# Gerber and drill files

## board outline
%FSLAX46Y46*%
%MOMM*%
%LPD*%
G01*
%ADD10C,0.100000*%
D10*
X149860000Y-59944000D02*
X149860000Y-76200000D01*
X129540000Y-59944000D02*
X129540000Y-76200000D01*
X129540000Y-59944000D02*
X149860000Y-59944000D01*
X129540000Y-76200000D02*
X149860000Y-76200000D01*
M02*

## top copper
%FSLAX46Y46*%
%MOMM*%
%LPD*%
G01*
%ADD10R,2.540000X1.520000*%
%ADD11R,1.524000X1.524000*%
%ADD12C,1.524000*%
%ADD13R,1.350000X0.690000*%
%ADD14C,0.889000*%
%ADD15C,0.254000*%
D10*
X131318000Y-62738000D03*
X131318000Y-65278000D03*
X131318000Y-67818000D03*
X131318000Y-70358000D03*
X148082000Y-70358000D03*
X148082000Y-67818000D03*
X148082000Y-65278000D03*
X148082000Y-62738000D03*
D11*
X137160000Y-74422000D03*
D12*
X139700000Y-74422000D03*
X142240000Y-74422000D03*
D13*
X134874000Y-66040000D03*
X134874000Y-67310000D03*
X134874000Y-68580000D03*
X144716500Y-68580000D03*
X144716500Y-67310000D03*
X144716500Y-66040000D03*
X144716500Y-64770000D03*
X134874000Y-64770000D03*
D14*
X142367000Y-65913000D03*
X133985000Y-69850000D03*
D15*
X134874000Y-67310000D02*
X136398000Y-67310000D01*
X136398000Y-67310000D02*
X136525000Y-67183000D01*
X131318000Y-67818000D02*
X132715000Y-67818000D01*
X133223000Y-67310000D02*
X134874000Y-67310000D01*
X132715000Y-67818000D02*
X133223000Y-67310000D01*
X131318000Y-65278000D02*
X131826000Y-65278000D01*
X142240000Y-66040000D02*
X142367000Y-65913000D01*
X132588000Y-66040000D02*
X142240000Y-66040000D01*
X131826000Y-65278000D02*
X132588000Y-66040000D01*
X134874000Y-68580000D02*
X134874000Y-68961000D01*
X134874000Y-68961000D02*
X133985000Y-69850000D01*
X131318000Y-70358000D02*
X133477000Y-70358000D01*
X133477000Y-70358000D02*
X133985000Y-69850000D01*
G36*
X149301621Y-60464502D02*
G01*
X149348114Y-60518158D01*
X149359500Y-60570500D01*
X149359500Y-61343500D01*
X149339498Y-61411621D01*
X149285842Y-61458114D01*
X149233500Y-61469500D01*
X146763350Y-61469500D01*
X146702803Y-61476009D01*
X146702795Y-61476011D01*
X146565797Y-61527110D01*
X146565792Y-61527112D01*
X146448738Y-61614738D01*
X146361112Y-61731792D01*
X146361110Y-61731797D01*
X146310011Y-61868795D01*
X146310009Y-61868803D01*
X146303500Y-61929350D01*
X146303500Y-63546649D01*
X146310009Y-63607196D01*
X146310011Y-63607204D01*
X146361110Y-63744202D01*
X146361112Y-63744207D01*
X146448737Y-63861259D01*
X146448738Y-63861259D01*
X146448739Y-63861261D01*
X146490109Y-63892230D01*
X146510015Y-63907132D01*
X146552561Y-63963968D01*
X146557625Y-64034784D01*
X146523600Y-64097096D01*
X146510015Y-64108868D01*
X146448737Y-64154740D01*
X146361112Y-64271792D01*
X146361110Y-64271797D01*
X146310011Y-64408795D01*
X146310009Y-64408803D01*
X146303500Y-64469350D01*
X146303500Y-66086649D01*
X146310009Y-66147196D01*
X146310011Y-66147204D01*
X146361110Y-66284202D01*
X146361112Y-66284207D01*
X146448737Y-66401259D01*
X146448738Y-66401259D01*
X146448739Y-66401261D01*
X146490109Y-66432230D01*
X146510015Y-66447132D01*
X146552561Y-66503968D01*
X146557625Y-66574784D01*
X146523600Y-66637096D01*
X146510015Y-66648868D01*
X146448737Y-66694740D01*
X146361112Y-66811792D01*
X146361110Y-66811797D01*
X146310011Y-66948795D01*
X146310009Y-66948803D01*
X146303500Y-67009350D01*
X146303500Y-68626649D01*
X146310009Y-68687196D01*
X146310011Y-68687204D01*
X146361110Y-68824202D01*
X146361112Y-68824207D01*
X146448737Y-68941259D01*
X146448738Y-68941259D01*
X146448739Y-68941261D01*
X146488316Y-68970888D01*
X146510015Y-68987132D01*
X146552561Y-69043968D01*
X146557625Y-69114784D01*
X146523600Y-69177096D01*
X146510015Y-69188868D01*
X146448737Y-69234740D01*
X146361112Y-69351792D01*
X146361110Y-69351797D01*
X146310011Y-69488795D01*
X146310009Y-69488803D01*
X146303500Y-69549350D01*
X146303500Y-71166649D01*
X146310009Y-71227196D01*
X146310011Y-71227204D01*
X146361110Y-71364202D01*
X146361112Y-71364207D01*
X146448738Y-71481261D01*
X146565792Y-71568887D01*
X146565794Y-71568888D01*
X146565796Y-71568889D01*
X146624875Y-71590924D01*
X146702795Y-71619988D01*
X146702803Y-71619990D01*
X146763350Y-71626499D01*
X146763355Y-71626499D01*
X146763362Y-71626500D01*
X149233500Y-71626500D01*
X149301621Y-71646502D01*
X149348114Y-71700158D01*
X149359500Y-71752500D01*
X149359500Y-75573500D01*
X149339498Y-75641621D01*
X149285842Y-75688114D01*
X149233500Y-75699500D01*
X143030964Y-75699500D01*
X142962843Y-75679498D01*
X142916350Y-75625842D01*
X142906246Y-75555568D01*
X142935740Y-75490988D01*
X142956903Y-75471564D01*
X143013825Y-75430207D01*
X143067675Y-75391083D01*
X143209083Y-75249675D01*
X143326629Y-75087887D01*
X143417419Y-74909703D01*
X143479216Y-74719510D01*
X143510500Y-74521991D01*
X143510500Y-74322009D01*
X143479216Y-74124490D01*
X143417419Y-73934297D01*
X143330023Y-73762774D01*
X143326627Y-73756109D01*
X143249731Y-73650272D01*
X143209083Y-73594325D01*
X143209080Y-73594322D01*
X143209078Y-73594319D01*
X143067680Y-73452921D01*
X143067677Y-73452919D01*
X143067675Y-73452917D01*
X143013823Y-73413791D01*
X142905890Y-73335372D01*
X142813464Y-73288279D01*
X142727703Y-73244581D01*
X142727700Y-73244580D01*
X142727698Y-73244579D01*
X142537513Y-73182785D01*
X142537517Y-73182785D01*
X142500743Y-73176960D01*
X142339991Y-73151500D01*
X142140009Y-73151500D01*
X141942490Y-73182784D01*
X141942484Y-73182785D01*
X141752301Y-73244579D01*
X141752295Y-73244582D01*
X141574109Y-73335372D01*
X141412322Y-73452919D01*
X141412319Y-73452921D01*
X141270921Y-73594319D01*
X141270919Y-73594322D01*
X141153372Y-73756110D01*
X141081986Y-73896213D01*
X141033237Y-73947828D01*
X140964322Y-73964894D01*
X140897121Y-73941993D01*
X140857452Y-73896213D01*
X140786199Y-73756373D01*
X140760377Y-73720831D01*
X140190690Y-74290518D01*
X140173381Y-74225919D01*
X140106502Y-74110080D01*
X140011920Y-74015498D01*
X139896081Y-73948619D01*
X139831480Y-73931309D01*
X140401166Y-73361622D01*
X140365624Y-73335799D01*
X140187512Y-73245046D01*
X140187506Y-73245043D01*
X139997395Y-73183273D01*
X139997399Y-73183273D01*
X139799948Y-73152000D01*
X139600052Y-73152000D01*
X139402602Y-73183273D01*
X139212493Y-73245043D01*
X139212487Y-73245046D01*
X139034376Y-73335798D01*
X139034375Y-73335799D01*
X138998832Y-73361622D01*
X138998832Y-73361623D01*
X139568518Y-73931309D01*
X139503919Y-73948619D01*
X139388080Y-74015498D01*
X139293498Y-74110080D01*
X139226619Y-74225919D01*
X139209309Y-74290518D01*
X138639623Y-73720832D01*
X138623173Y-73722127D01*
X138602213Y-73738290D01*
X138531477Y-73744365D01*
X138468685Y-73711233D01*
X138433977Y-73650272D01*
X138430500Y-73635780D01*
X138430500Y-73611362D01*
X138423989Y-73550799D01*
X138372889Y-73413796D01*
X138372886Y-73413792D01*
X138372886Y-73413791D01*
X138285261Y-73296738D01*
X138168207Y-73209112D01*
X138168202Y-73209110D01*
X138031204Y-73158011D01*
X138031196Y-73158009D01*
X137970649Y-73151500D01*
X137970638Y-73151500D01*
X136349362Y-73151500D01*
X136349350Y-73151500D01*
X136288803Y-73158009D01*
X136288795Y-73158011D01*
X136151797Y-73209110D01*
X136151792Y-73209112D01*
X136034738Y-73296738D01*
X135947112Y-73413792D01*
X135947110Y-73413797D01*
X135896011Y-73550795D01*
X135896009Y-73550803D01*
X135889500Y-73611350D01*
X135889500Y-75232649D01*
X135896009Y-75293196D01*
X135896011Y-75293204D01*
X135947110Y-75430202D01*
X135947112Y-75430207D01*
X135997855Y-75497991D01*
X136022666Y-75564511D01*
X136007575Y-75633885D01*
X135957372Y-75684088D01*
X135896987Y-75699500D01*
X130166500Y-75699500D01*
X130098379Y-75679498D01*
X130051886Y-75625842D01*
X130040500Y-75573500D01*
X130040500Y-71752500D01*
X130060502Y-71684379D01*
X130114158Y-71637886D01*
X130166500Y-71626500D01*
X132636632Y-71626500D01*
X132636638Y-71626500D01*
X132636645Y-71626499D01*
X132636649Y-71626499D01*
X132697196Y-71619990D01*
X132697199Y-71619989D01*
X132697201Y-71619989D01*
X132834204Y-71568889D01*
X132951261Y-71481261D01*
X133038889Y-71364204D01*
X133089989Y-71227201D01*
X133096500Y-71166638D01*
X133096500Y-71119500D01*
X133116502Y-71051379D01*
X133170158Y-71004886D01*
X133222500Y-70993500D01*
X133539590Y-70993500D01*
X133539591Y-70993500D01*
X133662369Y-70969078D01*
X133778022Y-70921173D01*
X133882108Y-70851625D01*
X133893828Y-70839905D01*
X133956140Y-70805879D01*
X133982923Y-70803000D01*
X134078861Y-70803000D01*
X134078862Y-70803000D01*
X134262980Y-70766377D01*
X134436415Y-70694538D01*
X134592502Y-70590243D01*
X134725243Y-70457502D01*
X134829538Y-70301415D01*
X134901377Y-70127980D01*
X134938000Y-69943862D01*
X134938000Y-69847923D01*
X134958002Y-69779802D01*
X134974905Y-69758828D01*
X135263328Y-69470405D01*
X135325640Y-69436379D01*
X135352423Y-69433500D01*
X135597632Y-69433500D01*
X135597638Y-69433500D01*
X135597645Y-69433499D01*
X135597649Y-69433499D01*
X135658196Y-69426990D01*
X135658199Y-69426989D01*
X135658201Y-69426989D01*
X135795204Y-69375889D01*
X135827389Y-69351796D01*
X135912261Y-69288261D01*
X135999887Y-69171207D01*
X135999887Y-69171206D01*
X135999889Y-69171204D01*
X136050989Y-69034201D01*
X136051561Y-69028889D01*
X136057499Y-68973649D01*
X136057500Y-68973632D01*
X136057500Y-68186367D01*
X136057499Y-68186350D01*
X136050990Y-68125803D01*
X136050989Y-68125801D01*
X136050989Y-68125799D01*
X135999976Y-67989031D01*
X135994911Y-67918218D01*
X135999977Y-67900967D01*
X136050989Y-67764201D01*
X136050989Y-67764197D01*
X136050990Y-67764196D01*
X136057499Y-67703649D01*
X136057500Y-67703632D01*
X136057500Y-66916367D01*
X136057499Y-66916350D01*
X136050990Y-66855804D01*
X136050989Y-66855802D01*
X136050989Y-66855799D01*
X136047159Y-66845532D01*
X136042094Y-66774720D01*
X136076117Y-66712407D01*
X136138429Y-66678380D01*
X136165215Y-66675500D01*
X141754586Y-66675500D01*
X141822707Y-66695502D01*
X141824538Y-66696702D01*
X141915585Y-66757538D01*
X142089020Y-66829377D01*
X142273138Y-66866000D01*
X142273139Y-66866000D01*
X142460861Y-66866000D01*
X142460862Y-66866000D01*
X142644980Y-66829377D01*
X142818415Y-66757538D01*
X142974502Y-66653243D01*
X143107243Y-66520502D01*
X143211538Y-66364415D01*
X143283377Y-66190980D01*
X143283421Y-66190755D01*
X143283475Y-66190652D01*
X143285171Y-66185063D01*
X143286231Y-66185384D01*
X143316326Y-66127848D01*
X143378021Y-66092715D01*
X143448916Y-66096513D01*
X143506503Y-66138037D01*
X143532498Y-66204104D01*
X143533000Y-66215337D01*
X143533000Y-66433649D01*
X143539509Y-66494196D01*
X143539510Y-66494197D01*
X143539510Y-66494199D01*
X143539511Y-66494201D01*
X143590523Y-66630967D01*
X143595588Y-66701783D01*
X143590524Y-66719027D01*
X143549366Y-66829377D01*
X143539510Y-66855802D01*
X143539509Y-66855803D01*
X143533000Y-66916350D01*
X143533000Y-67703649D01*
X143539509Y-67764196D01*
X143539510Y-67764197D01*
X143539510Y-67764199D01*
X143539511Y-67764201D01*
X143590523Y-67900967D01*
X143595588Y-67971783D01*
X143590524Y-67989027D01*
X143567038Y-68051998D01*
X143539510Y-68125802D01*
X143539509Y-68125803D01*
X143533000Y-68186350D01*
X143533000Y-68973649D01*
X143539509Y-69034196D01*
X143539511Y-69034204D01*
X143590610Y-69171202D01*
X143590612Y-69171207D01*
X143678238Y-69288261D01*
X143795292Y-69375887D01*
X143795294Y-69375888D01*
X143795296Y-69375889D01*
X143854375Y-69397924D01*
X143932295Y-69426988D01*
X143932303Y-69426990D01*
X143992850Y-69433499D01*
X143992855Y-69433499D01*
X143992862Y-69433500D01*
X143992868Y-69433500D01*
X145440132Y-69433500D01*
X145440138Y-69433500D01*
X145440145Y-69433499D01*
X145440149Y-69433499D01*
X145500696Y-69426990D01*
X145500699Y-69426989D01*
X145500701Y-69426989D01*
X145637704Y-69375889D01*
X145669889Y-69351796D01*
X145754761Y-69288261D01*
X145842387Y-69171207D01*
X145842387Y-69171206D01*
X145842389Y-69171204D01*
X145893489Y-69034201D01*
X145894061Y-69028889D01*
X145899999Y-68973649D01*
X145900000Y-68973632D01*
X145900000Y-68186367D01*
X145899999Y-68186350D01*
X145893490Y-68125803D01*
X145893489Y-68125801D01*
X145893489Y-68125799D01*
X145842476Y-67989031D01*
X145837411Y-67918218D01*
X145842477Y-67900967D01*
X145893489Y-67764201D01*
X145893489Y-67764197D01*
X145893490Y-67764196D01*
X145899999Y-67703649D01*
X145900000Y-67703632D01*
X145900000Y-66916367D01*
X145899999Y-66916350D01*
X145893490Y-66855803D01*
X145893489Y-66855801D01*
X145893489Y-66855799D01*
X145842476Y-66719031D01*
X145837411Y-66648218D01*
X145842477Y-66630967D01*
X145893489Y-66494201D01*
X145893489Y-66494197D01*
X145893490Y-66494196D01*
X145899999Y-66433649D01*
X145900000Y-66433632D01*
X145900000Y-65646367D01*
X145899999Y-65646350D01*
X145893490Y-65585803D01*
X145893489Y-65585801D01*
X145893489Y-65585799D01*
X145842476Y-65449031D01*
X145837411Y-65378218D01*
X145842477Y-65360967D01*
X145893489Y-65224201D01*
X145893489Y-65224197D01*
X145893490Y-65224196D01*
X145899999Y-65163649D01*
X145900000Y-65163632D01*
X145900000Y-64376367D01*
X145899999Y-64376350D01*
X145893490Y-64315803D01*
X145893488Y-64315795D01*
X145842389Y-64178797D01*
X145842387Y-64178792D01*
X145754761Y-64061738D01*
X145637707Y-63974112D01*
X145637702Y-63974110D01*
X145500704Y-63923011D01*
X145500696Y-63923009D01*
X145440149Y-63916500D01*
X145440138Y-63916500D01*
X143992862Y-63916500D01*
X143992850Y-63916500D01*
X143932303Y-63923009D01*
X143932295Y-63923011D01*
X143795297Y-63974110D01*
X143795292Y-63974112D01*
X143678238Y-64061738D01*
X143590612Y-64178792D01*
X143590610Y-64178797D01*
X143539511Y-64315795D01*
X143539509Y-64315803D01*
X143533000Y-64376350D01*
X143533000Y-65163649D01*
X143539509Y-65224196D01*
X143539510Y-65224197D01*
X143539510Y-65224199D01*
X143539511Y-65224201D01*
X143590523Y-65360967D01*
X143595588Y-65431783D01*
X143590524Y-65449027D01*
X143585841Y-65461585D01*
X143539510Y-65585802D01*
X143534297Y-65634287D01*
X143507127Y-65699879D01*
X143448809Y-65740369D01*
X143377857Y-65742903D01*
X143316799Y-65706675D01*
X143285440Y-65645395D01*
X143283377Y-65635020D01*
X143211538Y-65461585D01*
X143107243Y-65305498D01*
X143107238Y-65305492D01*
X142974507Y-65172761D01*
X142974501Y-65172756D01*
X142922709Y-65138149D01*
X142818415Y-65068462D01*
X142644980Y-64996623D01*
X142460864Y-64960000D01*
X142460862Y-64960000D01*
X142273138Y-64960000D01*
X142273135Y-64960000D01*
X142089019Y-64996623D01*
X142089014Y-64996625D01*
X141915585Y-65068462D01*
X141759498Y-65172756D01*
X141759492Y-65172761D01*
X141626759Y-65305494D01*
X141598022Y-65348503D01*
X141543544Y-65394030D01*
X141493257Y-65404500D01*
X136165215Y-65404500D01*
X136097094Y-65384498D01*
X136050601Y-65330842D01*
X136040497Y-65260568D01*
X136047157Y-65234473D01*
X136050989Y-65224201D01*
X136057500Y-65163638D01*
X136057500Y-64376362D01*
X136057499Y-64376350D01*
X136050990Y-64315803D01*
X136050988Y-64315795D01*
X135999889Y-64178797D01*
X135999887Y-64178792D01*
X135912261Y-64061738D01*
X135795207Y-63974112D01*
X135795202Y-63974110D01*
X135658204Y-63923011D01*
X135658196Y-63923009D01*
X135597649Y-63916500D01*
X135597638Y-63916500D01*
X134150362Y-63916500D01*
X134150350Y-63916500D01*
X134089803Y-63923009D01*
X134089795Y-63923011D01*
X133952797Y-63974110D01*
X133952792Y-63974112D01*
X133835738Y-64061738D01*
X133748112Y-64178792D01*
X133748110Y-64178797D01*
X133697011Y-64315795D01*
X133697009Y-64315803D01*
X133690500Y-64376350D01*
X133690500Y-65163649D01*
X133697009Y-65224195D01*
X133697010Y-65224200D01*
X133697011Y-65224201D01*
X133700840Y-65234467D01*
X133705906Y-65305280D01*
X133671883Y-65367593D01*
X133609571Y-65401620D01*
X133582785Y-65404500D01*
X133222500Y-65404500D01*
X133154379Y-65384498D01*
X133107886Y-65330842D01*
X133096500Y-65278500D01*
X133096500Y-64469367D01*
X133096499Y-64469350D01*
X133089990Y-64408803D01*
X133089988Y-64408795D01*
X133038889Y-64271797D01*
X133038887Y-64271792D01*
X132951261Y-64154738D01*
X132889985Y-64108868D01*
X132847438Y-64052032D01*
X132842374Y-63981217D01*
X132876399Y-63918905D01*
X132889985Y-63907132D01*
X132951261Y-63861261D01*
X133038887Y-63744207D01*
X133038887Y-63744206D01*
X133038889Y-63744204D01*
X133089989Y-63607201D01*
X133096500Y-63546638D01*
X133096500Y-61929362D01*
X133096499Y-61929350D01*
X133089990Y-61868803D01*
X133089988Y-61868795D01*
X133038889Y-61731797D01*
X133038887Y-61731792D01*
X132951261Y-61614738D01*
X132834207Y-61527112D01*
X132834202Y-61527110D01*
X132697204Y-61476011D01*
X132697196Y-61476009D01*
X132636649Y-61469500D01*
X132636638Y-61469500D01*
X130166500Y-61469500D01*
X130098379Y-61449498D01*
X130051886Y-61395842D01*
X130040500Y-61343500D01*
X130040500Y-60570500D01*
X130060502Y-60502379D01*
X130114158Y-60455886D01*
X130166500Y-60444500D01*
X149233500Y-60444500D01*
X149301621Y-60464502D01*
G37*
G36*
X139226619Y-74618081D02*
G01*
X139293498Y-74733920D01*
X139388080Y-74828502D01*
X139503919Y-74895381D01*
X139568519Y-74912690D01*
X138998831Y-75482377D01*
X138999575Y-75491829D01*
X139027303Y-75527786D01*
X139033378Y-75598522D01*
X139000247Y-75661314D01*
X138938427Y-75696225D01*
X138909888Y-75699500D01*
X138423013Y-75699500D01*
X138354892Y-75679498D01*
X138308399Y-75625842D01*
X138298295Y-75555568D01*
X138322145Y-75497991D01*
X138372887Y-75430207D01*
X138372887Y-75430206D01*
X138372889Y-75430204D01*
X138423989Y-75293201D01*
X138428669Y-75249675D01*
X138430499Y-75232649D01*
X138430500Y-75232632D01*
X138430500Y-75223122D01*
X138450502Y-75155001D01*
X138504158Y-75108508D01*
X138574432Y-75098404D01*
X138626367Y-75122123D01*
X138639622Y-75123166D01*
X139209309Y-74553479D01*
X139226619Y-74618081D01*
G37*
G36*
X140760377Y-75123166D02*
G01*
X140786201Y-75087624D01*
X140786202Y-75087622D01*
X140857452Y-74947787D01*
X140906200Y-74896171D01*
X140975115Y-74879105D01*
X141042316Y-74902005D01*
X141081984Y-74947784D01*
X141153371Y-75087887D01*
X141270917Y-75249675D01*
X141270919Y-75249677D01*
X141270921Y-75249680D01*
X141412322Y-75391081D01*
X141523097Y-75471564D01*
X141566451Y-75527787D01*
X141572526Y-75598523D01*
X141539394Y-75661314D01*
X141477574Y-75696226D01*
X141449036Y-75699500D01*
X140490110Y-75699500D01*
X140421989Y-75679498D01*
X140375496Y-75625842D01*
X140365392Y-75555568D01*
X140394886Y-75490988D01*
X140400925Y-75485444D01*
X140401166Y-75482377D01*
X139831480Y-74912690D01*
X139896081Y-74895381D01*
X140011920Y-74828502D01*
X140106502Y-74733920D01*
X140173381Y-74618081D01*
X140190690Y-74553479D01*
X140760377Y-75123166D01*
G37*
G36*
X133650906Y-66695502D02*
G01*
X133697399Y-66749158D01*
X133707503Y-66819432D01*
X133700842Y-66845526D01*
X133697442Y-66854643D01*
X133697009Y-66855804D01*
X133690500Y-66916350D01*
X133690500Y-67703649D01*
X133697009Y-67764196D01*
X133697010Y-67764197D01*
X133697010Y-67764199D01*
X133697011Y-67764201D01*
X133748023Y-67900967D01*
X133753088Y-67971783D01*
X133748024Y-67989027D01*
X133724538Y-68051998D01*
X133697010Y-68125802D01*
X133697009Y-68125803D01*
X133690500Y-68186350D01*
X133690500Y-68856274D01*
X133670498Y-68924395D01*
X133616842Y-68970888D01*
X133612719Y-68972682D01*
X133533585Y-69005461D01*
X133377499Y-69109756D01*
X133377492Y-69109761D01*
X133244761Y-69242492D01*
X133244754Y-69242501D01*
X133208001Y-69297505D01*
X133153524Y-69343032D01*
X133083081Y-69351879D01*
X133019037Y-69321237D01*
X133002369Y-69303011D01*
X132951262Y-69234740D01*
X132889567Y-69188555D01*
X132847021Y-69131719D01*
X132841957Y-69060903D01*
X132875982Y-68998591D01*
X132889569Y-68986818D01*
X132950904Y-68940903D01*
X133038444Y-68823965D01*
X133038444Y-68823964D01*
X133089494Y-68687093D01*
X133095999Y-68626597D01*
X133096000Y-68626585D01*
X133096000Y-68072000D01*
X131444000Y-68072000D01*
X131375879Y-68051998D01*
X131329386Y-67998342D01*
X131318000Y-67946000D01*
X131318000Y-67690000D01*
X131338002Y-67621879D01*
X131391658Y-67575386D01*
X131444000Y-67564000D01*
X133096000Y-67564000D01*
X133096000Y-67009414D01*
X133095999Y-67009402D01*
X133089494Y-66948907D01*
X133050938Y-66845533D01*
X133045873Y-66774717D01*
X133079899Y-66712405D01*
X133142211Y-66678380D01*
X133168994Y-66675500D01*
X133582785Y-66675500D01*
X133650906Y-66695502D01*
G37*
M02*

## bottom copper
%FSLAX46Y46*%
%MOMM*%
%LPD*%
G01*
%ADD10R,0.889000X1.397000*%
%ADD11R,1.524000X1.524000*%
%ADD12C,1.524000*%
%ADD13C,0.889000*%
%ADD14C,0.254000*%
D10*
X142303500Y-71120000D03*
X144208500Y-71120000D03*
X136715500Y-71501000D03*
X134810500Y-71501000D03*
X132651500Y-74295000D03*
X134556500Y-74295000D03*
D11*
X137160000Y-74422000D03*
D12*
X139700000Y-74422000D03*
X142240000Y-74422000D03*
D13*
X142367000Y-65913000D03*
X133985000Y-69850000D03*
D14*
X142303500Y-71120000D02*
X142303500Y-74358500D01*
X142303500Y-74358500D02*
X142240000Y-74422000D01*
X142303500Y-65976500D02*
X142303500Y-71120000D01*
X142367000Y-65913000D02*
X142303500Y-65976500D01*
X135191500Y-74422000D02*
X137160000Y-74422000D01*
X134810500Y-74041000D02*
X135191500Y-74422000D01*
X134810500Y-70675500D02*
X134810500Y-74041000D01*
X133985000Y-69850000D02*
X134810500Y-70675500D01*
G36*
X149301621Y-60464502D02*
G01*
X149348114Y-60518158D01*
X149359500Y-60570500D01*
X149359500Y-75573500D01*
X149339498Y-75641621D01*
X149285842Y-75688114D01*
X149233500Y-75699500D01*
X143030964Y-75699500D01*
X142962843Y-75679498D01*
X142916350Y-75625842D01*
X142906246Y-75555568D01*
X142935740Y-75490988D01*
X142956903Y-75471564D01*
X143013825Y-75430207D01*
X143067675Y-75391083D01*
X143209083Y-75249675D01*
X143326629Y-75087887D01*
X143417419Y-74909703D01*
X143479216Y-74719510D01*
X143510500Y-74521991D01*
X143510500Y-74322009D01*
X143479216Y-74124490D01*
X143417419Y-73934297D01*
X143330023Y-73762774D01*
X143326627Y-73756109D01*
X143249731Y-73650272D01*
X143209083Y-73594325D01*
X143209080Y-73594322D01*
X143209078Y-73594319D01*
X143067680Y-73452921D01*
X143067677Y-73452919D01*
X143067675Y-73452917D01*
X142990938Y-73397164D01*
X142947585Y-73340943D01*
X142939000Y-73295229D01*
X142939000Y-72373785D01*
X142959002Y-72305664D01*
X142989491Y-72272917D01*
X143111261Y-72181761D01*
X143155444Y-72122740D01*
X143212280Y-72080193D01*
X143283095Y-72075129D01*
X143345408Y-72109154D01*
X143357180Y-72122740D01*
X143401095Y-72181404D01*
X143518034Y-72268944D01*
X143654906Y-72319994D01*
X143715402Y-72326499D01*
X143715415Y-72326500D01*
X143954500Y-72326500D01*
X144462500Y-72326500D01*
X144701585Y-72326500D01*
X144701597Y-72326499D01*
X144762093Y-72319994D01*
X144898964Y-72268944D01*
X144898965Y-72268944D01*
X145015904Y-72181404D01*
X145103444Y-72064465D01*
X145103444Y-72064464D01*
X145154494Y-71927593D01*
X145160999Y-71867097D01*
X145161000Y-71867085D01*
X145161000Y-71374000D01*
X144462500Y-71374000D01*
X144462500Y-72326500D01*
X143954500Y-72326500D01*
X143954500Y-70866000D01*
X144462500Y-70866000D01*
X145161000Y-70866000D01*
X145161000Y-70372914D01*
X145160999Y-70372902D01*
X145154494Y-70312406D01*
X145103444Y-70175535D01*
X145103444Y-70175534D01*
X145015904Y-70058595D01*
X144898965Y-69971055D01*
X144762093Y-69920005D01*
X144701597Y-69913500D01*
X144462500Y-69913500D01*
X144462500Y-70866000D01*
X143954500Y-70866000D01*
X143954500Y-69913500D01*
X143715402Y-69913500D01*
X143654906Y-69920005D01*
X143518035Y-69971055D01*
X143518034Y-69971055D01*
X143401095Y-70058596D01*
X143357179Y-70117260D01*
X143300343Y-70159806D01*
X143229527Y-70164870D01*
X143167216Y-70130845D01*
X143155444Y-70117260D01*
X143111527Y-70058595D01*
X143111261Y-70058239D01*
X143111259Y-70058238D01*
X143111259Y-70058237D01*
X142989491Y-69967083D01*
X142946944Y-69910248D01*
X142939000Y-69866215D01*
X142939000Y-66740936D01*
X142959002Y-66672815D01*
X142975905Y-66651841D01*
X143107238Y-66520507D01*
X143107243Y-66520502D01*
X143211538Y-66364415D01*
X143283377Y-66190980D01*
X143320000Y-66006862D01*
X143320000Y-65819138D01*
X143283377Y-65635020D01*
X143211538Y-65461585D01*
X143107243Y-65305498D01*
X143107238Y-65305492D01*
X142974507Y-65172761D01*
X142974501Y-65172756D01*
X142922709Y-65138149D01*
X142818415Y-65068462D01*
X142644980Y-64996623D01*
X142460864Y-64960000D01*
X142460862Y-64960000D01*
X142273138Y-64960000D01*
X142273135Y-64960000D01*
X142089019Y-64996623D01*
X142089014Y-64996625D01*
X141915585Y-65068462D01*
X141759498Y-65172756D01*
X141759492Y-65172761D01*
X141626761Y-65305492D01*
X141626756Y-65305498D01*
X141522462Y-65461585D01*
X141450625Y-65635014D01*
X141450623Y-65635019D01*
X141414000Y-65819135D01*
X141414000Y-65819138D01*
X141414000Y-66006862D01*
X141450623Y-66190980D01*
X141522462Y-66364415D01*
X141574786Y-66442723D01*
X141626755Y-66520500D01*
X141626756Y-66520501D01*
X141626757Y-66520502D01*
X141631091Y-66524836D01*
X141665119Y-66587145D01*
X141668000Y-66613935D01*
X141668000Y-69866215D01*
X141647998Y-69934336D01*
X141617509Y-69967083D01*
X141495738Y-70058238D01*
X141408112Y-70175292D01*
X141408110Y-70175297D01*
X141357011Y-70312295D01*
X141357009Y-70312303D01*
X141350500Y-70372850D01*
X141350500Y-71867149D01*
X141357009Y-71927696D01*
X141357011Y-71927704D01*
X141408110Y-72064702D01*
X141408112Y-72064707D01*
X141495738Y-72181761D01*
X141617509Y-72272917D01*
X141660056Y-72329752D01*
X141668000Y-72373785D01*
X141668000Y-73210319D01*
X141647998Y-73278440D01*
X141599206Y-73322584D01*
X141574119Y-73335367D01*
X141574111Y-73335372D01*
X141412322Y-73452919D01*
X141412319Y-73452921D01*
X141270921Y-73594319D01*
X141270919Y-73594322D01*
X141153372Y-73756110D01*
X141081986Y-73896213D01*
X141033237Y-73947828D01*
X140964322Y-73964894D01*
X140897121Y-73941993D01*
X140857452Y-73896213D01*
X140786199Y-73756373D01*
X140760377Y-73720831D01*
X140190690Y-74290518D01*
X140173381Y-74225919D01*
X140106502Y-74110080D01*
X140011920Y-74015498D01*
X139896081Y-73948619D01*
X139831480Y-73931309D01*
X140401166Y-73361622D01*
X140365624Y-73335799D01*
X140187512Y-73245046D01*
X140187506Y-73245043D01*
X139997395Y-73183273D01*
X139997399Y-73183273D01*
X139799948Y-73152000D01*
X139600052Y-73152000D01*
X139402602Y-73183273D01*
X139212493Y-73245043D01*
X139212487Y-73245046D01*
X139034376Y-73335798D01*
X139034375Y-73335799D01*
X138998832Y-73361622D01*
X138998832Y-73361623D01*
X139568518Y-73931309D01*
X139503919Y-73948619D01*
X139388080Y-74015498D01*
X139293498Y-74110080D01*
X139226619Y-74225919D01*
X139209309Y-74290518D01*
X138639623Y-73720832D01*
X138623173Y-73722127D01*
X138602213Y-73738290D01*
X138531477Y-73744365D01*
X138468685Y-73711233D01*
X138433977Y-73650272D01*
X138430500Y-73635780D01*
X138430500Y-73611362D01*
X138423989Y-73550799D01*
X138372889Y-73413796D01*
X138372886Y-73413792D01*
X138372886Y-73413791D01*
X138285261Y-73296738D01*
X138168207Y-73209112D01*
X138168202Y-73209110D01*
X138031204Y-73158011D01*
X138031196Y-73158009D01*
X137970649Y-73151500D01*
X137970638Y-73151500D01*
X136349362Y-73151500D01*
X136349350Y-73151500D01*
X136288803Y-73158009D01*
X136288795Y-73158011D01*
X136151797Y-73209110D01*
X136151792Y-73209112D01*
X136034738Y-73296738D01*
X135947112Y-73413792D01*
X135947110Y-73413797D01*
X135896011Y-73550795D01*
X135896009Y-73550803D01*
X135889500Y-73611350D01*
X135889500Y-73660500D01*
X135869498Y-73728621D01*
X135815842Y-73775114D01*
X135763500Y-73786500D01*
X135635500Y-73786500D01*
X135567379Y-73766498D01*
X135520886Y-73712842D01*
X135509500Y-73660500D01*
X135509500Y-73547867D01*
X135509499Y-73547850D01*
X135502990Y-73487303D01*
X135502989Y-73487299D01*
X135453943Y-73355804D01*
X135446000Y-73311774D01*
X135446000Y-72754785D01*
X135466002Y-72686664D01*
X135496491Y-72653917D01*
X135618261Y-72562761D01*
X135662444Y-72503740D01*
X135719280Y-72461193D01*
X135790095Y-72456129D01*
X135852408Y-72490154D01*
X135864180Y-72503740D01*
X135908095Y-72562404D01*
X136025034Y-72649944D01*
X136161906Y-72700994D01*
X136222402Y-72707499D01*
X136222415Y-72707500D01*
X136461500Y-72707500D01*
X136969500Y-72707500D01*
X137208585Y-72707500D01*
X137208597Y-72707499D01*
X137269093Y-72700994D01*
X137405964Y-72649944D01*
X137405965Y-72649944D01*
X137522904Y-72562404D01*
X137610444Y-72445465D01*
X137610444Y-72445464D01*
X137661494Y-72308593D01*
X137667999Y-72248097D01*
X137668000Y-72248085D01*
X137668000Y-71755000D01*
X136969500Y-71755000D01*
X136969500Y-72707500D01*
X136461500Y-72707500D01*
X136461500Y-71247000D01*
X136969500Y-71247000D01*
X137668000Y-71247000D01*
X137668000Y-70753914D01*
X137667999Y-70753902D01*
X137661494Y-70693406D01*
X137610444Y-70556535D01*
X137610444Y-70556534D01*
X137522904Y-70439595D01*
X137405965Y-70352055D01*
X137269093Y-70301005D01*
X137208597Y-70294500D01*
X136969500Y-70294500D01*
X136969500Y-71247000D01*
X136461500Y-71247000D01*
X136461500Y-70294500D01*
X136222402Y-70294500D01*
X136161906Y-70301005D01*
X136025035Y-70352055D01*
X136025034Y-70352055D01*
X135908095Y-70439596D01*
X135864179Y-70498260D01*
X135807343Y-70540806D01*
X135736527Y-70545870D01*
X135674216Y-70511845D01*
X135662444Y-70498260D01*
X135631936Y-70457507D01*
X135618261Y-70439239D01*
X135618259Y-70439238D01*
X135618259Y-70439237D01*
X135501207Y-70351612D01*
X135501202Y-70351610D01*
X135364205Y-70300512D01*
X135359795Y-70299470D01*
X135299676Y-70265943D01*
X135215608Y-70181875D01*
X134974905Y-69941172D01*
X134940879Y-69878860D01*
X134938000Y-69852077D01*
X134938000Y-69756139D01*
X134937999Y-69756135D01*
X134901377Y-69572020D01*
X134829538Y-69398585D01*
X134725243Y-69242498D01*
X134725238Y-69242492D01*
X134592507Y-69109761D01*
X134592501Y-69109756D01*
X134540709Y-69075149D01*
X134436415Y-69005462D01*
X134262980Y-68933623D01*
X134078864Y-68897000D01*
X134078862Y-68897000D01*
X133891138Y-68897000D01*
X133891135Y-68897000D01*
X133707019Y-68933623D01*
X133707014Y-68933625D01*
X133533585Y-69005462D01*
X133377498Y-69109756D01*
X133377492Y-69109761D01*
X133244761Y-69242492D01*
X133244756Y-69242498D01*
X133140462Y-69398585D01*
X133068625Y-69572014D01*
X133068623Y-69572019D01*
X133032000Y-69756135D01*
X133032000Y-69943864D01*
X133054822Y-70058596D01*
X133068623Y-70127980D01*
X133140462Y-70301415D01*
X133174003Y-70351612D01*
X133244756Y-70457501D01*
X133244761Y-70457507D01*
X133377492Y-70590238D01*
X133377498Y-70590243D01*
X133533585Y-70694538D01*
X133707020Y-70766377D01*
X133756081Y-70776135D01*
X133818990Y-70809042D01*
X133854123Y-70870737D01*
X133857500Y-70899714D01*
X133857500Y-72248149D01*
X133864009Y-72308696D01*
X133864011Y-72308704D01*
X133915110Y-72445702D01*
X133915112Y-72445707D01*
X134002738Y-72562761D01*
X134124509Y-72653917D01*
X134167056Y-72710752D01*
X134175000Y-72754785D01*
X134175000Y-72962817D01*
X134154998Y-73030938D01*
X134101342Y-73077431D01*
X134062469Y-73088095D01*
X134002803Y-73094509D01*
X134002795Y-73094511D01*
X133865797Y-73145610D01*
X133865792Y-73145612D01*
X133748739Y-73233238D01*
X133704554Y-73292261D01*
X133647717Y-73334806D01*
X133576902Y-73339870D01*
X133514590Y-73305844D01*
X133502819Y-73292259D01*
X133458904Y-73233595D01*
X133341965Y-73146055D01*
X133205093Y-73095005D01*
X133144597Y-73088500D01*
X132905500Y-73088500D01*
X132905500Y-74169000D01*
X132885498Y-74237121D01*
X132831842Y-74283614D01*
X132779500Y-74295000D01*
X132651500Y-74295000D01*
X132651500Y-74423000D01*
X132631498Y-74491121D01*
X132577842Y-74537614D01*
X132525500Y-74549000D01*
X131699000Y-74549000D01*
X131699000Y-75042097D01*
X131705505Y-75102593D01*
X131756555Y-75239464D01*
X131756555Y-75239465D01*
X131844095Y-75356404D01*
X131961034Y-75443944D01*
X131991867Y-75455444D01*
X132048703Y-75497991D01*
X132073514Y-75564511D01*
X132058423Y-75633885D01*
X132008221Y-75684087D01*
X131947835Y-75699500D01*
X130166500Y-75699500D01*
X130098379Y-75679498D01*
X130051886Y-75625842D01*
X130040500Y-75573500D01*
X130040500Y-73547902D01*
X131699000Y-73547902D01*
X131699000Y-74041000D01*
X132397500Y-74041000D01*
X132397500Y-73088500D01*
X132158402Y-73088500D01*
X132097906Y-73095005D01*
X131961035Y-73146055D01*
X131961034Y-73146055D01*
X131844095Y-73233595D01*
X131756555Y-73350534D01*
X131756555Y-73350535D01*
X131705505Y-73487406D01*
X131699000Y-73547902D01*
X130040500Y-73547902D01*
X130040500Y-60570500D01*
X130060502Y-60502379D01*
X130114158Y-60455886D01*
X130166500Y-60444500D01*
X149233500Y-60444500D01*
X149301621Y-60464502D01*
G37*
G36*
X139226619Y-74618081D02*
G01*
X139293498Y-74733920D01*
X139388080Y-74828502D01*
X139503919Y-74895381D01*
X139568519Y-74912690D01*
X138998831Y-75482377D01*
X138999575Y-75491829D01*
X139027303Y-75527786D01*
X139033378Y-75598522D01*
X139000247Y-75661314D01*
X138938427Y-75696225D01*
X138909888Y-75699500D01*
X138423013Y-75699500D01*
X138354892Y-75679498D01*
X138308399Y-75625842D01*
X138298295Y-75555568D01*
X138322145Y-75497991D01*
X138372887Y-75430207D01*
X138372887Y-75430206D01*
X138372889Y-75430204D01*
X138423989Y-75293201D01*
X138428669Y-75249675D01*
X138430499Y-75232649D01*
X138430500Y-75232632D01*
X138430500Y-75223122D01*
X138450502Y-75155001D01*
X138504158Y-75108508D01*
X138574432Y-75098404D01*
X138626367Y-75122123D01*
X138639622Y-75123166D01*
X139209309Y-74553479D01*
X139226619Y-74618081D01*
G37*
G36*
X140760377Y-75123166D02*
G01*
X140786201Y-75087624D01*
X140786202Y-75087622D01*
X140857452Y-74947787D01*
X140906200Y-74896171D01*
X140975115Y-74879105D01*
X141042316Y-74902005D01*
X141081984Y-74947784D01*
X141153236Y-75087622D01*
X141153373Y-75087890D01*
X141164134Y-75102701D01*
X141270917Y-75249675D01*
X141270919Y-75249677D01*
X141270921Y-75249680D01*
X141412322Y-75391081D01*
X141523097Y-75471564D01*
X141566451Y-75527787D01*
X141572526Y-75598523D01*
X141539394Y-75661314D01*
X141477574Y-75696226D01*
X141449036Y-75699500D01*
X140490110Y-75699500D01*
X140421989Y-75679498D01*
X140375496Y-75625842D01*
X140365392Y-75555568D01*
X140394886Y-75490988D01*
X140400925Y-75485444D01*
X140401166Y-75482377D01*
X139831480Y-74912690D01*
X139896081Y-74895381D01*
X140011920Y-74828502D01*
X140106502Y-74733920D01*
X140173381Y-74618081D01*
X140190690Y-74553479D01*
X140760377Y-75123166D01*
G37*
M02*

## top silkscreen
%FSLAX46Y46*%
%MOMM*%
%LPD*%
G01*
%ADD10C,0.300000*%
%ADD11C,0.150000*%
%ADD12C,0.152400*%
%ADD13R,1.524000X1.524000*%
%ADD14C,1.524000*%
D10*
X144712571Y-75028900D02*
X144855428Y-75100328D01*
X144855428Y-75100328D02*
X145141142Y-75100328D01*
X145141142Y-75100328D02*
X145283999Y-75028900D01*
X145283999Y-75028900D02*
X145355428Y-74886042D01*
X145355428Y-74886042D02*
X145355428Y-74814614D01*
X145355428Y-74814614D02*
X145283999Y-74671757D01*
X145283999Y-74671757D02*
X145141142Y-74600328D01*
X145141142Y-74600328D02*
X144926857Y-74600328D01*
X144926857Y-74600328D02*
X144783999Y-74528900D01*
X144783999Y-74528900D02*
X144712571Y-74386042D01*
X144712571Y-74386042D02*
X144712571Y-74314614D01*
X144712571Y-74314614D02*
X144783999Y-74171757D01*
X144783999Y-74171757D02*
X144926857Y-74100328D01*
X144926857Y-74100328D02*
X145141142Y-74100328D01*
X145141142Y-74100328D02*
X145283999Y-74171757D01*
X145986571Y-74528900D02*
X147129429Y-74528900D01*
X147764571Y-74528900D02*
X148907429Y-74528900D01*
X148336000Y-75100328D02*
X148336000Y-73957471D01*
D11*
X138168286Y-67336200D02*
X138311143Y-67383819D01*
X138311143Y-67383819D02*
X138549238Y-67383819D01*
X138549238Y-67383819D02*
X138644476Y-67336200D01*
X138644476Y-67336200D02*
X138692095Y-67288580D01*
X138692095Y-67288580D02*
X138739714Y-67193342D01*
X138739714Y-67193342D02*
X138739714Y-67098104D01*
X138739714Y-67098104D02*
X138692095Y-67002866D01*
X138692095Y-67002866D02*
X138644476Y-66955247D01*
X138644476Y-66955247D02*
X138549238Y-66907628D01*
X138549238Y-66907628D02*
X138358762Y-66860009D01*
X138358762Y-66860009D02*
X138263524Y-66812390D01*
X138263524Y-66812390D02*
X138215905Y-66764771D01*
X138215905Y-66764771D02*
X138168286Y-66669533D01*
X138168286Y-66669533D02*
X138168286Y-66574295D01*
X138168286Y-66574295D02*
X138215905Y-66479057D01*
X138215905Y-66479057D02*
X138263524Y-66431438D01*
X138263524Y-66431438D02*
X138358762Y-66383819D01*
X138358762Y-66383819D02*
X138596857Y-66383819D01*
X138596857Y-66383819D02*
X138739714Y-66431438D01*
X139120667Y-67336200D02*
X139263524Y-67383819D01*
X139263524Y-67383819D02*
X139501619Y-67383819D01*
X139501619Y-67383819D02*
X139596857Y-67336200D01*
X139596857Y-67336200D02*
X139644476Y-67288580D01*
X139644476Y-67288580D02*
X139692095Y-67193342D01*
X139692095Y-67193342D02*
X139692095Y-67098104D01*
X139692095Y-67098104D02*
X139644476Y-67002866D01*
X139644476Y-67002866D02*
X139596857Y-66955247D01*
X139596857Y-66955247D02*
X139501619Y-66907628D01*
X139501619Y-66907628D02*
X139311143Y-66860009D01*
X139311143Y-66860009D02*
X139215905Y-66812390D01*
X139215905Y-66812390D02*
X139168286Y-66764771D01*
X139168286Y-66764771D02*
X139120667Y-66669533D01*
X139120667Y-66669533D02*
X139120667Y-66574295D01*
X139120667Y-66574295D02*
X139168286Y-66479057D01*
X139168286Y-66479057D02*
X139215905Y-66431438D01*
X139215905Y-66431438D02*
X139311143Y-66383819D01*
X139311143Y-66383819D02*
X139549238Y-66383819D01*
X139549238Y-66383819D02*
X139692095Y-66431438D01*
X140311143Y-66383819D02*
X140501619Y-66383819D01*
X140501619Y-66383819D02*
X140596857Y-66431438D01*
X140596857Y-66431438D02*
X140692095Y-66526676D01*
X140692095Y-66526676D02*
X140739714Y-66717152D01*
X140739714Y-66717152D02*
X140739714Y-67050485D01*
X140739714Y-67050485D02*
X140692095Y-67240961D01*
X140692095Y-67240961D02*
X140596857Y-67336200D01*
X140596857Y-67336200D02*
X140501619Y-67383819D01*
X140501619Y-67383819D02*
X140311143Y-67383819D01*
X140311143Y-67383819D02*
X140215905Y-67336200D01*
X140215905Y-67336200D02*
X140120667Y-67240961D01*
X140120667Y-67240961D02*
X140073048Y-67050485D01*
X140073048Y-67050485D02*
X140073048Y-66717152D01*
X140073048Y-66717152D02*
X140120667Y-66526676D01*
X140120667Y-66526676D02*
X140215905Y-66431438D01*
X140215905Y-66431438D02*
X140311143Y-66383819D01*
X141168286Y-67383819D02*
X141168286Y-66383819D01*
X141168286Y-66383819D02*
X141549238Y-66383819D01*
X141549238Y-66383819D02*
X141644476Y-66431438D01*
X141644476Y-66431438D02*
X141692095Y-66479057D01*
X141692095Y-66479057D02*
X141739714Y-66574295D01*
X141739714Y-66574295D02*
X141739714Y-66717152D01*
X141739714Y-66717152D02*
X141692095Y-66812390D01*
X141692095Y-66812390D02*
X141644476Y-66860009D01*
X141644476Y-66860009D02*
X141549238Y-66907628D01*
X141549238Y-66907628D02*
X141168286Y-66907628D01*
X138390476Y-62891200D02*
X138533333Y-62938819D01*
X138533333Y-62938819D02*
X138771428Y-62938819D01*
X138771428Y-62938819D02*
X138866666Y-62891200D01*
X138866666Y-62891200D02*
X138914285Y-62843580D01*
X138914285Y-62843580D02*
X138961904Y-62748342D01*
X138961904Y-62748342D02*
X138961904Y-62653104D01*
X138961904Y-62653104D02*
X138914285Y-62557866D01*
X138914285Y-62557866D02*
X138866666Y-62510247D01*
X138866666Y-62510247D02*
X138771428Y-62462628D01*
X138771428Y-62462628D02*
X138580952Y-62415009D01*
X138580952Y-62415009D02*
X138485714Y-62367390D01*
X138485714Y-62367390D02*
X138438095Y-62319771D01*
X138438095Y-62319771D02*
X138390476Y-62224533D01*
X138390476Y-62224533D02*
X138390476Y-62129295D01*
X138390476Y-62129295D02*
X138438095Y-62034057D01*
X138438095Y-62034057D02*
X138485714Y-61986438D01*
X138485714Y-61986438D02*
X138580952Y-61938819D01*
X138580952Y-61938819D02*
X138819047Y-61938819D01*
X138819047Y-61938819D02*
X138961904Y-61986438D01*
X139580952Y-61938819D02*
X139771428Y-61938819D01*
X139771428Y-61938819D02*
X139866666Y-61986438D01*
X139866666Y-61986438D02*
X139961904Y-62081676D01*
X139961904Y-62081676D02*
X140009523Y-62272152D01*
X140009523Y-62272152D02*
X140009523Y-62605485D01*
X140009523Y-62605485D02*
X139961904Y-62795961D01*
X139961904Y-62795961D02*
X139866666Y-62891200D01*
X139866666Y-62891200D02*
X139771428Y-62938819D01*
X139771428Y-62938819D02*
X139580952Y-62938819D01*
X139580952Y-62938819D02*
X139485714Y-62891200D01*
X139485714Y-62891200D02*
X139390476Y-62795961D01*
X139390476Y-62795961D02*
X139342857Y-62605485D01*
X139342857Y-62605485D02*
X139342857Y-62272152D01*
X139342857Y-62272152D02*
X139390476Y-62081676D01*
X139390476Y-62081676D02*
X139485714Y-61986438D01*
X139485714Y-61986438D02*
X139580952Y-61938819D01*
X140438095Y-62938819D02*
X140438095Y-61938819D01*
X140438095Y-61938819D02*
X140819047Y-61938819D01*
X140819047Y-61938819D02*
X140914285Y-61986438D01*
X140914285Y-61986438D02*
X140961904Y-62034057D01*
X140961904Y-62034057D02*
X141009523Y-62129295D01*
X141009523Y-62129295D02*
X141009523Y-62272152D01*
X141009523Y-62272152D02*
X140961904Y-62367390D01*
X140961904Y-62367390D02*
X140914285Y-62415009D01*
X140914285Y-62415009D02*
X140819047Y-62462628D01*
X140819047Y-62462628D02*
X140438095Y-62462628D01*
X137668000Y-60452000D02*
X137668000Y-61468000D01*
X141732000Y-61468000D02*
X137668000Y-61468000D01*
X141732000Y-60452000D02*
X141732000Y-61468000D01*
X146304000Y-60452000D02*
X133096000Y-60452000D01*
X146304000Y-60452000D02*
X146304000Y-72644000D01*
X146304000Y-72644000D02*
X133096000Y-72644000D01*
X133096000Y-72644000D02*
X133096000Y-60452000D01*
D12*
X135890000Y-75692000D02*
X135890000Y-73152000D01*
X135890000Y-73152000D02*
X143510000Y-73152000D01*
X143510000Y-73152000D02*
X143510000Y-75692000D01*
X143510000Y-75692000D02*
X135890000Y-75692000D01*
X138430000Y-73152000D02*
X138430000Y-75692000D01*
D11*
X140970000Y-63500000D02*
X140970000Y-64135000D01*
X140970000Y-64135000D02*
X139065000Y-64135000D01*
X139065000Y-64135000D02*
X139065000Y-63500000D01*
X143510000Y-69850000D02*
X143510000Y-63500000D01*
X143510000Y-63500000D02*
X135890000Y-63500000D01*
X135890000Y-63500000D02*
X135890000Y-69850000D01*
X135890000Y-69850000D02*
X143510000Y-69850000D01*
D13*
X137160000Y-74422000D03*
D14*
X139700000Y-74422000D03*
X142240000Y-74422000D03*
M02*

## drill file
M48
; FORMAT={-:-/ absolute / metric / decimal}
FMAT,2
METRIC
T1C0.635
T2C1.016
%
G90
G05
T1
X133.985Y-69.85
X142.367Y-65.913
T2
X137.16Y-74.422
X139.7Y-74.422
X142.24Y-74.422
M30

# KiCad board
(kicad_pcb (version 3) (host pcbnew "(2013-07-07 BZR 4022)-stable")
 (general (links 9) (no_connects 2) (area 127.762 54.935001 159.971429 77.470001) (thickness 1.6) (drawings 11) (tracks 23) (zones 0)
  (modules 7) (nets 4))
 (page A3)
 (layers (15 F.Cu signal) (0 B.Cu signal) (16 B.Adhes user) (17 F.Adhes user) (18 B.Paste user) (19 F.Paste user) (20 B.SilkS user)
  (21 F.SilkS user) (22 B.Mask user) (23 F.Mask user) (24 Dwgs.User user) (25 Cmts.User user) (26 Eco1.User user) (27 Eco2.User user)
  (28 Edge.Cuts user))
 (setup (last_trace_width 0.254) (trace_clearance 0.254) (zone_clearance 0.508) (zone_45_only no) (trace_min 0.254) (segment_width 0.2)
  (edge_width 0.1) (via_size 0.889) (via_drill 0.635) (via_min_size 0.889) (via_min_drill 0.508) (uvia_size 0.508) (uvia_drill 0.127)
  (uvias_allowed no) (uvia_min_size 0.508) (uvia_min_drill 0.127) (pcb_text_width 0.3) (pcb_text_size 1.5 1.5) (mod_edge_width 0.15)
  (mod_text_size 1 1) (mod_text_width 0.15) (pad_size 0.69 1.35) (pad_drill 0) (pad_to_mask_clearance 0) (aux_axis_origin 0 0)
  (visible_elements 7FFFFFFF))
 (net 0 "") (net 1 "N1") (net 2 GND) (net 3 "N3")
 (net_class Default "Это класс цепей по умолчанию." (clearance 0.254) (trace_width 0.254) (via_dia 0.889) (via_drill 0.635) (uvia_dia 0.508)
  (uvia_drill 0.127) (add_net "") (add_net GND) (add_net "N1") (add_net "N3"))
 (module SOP (layer F.Cu) (at 139.7 66.548)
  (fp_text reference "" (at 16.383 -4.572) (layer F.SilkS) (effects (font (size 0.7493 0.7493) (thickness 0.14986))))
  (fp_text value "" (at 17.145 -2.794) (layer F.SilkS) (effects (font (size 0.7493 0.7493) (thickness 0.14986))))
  (fp_line (start -2.032 -6.096) (end -2.032 -5.08) (layer F.SilkS) (width 0.15))
  (fp_line (start 2.032 -5.08) (end -2.032 -5.08) (layer F.SilkS) (width 0.15))
  (fp_line (start 2.032 -6.096) (end 2.032 -5.08) (layer F.SilkS) (width 0.15))
  (fp_line (start 6.604 -6.096) (end -6.604 -6.096) (layer F.SilkS) (width 0.15))
  (fp_line (start 6.604 -6.096) (end 6.604 6.096) (layer F.SilkS) (width 0.15))
  (fp_line (start 6.604 6.096) (end -6.604 6.096) (layer F.SilkS) (width 0.15))
  (fp_line (start -6.604 6.096) (end -6.604 -6.096) (layer F.SilkS) (width 0.15))
  (pad 1 smd rect (at -8.382 -3.81 270) (size 1.52 2.54) (layers F.Cu F.Paste F.Mask))
  (pad 2 smd rect (at -8.382 -1.27 270) (size 1.52 2.54) (layers F.Cu F.Paste F.Mask) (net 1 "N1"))
  (pad 3 smd rect (at -8.382 1.27 270) (size 1.52 2.54) (layers F.Cu F.Paste F.Mask) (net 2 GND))
  (pad 4 smd rect (at -8.382 3.81 270) (size 1.52 2.54) (layers F.Cu F.Paste F.Mask) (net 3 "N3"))
  (pad 5 smd rect (at 8.382 3.81 270) (size 1.52 2.54) (layers F.Cu F.Paste F.Mask))
  (pad 6 smd rect (at 8.382 1.27 270) (size 1.52 2.54) (layers F.Cu F.Paste F.Mask))
  (pad 7 smd rect (at 8.382 -1.27 270) (size 1.52 2.54) (layers F.Cu F.Paste F.Mask))
  (pad 8 smd rect (at 8.382 -3.81 270) (size 1.52 2.54) (layers F.Cu F.Paste F.Mask)))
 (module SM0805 (layer B.Cu) (at 143.256 71.12)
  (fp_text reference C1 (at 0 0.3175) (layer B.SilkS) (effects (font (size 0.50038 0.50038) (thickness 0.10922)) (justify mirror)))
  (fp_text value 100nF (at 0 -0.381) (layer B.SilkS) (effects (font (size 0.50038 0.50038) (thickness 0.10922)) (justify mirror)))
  (pad 1 smd rect (at -0.9525 0) (size 0.889 1.397) (layers B.Cu B.Paste B.Mask) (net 1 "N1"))
  (pad 2 smd rect (at 0.9525 0) (size 0.889 1.397) (layers B.Cu B.Paste B.Mask) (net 2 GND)))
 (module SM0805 (layer B.Cu) (at 135.763 71.501 180)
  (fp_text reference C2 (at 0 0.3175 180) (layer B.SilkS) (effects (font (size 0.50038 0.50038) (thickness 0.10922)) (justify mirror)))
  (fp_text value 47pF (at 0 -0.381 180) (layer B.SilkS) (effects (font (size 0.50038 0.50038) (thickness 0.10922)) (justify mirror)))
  (pad 1 smd rect (at -0.9525 0 180) (size 0.889 1.397) (layers B.Cu B.Paste B.Mask) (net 2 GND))
  (pad 2 smd rect (at 0.9525 0 180) (size 0.889 1.397) (layers B.Cu B.Paste B.Mask) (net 3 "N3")))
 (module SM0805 (layer B.Cu) (at 133.604 74.295)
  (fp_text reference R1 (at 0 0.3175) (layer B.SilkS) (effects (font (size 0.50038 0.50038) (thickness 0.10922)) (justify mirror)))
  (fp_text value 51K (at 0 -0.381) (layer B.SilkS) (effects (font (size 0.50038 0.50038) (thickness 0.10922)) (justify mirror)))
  (pad 1 smd rect (at -0.9525 0) (size 0.889 1.397) (layers B.Cu B.Paste B.Mask) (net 2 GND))
  (pad 2 smd rect (at 0.9525 0) (size 0.889 1.397) (layers B.Cu B.Paste B.Mask) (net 3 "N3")))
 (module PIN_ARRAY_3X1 (layer F.Cu) (at 139.7 74.422)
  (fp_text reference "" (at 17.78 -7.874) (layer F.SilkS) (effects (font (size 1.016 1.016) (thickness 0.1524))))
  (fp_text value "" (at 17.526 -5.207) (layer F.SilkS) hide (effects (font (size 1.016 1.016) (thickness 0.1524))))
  (fp_line (start -3.81 1.27) (end -3.81 -1.27) (layer F.SilkS) (width 0.1524))
  (fp_line (start -3.81 -1.27) (end 3.81 -1.27) (layer F.SilkS) (width 0.1524))
  (fp_line (start 3.81 -1.27) (end 3.81 1.27) (layer F.SilkS) (width 0.1524))
  (fp_line (start 3.81 1.27) (end -3.81 1.27) (layer F.SilkS) (width 0.1524))
  (fp_line (start -1.27 -1.27) (end -1.27 1.27) (layer F.SilkS) (width 0.1524))
  (pad 1 thru_hole rect (at -2.54 0) (size 1.524 1.524) (drill 1.016) (layers *.Cu *.Mask F.SilkS) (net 3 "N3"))
  (pad 2 thru_hole circle (at 0 0) (size 1.524 1.524) (drill 1.016) (layers *.Cu *.Mask F.SilkS) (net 2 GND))
  (pad 3 thru_hole circle (at 2.54 0) (size 1.524 1.524) (drill 1.016) (layers *.Cu *.Mask F.SilkS) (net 1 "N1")))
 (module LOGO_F (layer B.Cu) (at 146.177 66.675)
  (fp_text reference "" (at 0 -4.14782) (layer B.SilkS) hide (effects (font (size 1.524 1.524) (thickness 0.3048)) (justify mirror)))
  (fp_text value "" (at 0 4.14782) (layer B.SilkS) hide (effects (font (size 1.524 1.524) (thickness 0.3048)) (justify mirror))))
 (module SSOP (layer F.Cu) (at 139.7 66.675)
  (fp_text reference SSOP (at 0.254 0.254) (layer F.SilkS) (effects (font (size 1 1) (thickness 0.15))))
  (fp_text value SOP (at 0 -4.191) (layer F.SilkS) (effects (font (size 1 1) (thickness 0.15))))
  (fp_line (start 1.27 -3.175) (end 1.27 -2.54) (layer F.SilkS) (width 0.15))
  (fp_line (start 1.27 -2.54) (end -0.635 -2.54) (layer F.SilkS) (width 0.15))
  (fp_line (start -0.635 -2.54) (end -0.635 -3.175) (layer F.SilkS) (width 0.15))
  (fp_line (start 3.81 3.175) (end 3.81 -3.175) (layer F.SilkS) (width 0.15))
  (fp_line (start 3.81 -3.175) (end -3.81 -3.175) (layer F.SilkS) (width 0.15))
  (fp_line (start -3.81 -3.175) (end -3.81 3.175) (layer F.SilkS) (width 0.15))
  (fp_line (start -3.81 3.175) (end 3.81 3.175) (layer F.SilkS) (width 0.15))
  (pad 2 smd rect (at -4.826 -0.635 270) (size 0.69 1.35) (layers F.Cu F.Paste F.Mask))
  (pad 3 smd rect (at -4.826 0.635 270) (size 0.69 1.35) (layers F.Cu F.Paste F.Mask))
  (pad 4 smd rect (at -4.826 1.905 270) (size 0.69 1.35) (layers F.Cu F.Paste F.Mask))
  (pad 5 smd rect (at 5.0165 1.905 270) (size 0.69 1.35) (layers F.Cu F.Paste F.Mask))
  (pad 6 smd rect (at 5.0165 0.635 270) (size 0.69 1.35) (layers F.Cu F.Paste F.Mask))
  (pad 7 smd rect (at 5.0165 -0.635 270) (size 0.69 1.35) (layers F.Cu F.Paste F.Mask))
  (pad 8 smd rect (at 5.0165 -1.905 270) (size 0.69 1.35) (layers F.Cu F.Paste F.Mask))
  (pad 1 smd rect (at -4.826 -1.905 270) (size 0.69 1.35) (layers F.Cu F.Paste F.Mask)))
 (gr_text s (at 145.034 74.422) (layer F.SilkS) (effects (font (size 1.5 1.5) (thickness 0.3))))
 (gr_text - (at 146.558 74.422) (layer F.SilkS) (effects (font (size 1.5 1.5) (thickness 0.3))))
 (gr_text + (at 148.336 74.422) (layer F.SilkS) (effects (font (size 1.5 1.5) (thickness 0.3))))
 (gr_line (start 149.86 59.944) (end 149.86 76.2) (angle 90) (layer Edge.Cuts) (width 0.1))
 (gr_line (start 129.54 59.944) (end 129.54 76.2) (angle 90) (layer Edge.Cuts) (width 0.1))
 (gr_line (start 129.54 59.944) (end 149.86 59.944) (angle 90) (layer Edge.Cuts) (width 0.1))
 (gr_line (start 129.54 76.2) (end 149.86 76.2) (angle 90) (layer Edge.Cuts) (width 0.1))
 (segment (start 134.874 67.31) (end 136.398 67.31) (width 0.254) (layer F.Cu) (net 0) (status 400000))
 (segment (start 136.398 67.31) (end 136.525 67.183) (width 0.254) (layer F.Cu) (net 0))
 (segment (start 131.318 67.818) (end 132.715 67.818) (width 0.254) (layer F.Cu) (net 2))
 (segment (start 133.223 67.31) (end 134.874 67.31) (width 0.254) (layer F.Cu) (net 2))
 (segment (start 132.715 67.818) (end 133.223 67.31) (width 0.254) (layer F.Cu) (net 2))
 (segment (start 142.3035 71.12) (end 142.3035 74.3585) (width 0.254) (layer B.Cu) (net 1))
 (segment (start 142.3035 74.3585) (end 142.24 74.422) (width 0.254) (layer B.Cu) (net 1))
 (segment (start 131.318 65.278) (end 131.826 65.278) (width 0.254) (layer F.Cu) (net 1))
 (segment (start 142.3035 65.9765) (end 142.3035 71.12) (width 0.254) (layer B.Cu) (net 1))
 (segment (start 142.367 65.913) (end 142.3035 65.9765) (width 0.254) (layer B.Cu) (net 1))
 (via (at 142.367 65.913) (size 0.889) (layers F.Cu B.Cu) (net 1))
 (segment (start 142.24 66.04) (end 142.367 65.913) (width 0.254) (layer F.Cu) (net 1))
 (segment (start 132.588 66.04) (end 142.24 66.04) (width 0.254) (layer F.Cu) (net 1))
 (segment (start 131.826 65.278) (end 132.588 66.04) (width 0.254) (layer F.Cu) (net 1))
 (segment (start 134.874 68.58) (end 134.874 68.961) (width 0.254) (layer F.Cu) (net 3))
 (segment (start 134.874 68.961) (end 133.985 69.85) (width 0.254) (layer F.Cu) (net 3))
 (segment (start 131.318 70.358) (end 133.477 70.358) (width 0.254) (layer F.Cu) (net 3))
 (segment (start 135.1915 74.422) (end 137.16 74.422) (width 0.254) (layer B.Cu) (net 3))
 (segment (start 134.8105 74.041) (end 135.1915 74.422) (width 0.254) (layer B.Cu) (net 3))
 (segment (start 134.8105 70.6755) (end 134.8105 74.041) (width 0.254) (layer B.Cu) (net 3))
 (segment (start 133.985 69.85) (end 134.8105 70.6755) (width 0.254) (layer B.Cu) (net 3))
 (via (at 133.985 69.85) (size 0.889) (layers F.Cu B.Cu) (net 3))
 (segment (start 133.477 70.358) (end 133.985 69.85) (width 0.254) (layer F.Cu) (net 3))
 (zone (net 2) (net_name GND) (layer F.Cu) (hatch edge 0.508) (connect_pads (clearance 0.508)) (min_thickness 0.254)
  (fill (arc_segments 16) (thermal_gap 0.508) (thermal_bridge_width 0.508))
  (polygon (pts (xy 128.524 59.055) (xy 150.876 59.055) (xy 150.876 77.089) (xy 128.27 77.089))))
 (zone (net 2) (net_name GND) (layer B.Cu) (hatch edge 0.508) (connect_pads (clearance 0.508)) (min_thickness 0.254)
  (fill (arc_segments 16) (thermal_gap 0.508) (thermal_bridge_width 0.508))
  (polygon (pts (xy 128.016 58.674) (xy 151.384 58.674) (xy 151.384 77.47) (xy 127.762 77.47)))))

